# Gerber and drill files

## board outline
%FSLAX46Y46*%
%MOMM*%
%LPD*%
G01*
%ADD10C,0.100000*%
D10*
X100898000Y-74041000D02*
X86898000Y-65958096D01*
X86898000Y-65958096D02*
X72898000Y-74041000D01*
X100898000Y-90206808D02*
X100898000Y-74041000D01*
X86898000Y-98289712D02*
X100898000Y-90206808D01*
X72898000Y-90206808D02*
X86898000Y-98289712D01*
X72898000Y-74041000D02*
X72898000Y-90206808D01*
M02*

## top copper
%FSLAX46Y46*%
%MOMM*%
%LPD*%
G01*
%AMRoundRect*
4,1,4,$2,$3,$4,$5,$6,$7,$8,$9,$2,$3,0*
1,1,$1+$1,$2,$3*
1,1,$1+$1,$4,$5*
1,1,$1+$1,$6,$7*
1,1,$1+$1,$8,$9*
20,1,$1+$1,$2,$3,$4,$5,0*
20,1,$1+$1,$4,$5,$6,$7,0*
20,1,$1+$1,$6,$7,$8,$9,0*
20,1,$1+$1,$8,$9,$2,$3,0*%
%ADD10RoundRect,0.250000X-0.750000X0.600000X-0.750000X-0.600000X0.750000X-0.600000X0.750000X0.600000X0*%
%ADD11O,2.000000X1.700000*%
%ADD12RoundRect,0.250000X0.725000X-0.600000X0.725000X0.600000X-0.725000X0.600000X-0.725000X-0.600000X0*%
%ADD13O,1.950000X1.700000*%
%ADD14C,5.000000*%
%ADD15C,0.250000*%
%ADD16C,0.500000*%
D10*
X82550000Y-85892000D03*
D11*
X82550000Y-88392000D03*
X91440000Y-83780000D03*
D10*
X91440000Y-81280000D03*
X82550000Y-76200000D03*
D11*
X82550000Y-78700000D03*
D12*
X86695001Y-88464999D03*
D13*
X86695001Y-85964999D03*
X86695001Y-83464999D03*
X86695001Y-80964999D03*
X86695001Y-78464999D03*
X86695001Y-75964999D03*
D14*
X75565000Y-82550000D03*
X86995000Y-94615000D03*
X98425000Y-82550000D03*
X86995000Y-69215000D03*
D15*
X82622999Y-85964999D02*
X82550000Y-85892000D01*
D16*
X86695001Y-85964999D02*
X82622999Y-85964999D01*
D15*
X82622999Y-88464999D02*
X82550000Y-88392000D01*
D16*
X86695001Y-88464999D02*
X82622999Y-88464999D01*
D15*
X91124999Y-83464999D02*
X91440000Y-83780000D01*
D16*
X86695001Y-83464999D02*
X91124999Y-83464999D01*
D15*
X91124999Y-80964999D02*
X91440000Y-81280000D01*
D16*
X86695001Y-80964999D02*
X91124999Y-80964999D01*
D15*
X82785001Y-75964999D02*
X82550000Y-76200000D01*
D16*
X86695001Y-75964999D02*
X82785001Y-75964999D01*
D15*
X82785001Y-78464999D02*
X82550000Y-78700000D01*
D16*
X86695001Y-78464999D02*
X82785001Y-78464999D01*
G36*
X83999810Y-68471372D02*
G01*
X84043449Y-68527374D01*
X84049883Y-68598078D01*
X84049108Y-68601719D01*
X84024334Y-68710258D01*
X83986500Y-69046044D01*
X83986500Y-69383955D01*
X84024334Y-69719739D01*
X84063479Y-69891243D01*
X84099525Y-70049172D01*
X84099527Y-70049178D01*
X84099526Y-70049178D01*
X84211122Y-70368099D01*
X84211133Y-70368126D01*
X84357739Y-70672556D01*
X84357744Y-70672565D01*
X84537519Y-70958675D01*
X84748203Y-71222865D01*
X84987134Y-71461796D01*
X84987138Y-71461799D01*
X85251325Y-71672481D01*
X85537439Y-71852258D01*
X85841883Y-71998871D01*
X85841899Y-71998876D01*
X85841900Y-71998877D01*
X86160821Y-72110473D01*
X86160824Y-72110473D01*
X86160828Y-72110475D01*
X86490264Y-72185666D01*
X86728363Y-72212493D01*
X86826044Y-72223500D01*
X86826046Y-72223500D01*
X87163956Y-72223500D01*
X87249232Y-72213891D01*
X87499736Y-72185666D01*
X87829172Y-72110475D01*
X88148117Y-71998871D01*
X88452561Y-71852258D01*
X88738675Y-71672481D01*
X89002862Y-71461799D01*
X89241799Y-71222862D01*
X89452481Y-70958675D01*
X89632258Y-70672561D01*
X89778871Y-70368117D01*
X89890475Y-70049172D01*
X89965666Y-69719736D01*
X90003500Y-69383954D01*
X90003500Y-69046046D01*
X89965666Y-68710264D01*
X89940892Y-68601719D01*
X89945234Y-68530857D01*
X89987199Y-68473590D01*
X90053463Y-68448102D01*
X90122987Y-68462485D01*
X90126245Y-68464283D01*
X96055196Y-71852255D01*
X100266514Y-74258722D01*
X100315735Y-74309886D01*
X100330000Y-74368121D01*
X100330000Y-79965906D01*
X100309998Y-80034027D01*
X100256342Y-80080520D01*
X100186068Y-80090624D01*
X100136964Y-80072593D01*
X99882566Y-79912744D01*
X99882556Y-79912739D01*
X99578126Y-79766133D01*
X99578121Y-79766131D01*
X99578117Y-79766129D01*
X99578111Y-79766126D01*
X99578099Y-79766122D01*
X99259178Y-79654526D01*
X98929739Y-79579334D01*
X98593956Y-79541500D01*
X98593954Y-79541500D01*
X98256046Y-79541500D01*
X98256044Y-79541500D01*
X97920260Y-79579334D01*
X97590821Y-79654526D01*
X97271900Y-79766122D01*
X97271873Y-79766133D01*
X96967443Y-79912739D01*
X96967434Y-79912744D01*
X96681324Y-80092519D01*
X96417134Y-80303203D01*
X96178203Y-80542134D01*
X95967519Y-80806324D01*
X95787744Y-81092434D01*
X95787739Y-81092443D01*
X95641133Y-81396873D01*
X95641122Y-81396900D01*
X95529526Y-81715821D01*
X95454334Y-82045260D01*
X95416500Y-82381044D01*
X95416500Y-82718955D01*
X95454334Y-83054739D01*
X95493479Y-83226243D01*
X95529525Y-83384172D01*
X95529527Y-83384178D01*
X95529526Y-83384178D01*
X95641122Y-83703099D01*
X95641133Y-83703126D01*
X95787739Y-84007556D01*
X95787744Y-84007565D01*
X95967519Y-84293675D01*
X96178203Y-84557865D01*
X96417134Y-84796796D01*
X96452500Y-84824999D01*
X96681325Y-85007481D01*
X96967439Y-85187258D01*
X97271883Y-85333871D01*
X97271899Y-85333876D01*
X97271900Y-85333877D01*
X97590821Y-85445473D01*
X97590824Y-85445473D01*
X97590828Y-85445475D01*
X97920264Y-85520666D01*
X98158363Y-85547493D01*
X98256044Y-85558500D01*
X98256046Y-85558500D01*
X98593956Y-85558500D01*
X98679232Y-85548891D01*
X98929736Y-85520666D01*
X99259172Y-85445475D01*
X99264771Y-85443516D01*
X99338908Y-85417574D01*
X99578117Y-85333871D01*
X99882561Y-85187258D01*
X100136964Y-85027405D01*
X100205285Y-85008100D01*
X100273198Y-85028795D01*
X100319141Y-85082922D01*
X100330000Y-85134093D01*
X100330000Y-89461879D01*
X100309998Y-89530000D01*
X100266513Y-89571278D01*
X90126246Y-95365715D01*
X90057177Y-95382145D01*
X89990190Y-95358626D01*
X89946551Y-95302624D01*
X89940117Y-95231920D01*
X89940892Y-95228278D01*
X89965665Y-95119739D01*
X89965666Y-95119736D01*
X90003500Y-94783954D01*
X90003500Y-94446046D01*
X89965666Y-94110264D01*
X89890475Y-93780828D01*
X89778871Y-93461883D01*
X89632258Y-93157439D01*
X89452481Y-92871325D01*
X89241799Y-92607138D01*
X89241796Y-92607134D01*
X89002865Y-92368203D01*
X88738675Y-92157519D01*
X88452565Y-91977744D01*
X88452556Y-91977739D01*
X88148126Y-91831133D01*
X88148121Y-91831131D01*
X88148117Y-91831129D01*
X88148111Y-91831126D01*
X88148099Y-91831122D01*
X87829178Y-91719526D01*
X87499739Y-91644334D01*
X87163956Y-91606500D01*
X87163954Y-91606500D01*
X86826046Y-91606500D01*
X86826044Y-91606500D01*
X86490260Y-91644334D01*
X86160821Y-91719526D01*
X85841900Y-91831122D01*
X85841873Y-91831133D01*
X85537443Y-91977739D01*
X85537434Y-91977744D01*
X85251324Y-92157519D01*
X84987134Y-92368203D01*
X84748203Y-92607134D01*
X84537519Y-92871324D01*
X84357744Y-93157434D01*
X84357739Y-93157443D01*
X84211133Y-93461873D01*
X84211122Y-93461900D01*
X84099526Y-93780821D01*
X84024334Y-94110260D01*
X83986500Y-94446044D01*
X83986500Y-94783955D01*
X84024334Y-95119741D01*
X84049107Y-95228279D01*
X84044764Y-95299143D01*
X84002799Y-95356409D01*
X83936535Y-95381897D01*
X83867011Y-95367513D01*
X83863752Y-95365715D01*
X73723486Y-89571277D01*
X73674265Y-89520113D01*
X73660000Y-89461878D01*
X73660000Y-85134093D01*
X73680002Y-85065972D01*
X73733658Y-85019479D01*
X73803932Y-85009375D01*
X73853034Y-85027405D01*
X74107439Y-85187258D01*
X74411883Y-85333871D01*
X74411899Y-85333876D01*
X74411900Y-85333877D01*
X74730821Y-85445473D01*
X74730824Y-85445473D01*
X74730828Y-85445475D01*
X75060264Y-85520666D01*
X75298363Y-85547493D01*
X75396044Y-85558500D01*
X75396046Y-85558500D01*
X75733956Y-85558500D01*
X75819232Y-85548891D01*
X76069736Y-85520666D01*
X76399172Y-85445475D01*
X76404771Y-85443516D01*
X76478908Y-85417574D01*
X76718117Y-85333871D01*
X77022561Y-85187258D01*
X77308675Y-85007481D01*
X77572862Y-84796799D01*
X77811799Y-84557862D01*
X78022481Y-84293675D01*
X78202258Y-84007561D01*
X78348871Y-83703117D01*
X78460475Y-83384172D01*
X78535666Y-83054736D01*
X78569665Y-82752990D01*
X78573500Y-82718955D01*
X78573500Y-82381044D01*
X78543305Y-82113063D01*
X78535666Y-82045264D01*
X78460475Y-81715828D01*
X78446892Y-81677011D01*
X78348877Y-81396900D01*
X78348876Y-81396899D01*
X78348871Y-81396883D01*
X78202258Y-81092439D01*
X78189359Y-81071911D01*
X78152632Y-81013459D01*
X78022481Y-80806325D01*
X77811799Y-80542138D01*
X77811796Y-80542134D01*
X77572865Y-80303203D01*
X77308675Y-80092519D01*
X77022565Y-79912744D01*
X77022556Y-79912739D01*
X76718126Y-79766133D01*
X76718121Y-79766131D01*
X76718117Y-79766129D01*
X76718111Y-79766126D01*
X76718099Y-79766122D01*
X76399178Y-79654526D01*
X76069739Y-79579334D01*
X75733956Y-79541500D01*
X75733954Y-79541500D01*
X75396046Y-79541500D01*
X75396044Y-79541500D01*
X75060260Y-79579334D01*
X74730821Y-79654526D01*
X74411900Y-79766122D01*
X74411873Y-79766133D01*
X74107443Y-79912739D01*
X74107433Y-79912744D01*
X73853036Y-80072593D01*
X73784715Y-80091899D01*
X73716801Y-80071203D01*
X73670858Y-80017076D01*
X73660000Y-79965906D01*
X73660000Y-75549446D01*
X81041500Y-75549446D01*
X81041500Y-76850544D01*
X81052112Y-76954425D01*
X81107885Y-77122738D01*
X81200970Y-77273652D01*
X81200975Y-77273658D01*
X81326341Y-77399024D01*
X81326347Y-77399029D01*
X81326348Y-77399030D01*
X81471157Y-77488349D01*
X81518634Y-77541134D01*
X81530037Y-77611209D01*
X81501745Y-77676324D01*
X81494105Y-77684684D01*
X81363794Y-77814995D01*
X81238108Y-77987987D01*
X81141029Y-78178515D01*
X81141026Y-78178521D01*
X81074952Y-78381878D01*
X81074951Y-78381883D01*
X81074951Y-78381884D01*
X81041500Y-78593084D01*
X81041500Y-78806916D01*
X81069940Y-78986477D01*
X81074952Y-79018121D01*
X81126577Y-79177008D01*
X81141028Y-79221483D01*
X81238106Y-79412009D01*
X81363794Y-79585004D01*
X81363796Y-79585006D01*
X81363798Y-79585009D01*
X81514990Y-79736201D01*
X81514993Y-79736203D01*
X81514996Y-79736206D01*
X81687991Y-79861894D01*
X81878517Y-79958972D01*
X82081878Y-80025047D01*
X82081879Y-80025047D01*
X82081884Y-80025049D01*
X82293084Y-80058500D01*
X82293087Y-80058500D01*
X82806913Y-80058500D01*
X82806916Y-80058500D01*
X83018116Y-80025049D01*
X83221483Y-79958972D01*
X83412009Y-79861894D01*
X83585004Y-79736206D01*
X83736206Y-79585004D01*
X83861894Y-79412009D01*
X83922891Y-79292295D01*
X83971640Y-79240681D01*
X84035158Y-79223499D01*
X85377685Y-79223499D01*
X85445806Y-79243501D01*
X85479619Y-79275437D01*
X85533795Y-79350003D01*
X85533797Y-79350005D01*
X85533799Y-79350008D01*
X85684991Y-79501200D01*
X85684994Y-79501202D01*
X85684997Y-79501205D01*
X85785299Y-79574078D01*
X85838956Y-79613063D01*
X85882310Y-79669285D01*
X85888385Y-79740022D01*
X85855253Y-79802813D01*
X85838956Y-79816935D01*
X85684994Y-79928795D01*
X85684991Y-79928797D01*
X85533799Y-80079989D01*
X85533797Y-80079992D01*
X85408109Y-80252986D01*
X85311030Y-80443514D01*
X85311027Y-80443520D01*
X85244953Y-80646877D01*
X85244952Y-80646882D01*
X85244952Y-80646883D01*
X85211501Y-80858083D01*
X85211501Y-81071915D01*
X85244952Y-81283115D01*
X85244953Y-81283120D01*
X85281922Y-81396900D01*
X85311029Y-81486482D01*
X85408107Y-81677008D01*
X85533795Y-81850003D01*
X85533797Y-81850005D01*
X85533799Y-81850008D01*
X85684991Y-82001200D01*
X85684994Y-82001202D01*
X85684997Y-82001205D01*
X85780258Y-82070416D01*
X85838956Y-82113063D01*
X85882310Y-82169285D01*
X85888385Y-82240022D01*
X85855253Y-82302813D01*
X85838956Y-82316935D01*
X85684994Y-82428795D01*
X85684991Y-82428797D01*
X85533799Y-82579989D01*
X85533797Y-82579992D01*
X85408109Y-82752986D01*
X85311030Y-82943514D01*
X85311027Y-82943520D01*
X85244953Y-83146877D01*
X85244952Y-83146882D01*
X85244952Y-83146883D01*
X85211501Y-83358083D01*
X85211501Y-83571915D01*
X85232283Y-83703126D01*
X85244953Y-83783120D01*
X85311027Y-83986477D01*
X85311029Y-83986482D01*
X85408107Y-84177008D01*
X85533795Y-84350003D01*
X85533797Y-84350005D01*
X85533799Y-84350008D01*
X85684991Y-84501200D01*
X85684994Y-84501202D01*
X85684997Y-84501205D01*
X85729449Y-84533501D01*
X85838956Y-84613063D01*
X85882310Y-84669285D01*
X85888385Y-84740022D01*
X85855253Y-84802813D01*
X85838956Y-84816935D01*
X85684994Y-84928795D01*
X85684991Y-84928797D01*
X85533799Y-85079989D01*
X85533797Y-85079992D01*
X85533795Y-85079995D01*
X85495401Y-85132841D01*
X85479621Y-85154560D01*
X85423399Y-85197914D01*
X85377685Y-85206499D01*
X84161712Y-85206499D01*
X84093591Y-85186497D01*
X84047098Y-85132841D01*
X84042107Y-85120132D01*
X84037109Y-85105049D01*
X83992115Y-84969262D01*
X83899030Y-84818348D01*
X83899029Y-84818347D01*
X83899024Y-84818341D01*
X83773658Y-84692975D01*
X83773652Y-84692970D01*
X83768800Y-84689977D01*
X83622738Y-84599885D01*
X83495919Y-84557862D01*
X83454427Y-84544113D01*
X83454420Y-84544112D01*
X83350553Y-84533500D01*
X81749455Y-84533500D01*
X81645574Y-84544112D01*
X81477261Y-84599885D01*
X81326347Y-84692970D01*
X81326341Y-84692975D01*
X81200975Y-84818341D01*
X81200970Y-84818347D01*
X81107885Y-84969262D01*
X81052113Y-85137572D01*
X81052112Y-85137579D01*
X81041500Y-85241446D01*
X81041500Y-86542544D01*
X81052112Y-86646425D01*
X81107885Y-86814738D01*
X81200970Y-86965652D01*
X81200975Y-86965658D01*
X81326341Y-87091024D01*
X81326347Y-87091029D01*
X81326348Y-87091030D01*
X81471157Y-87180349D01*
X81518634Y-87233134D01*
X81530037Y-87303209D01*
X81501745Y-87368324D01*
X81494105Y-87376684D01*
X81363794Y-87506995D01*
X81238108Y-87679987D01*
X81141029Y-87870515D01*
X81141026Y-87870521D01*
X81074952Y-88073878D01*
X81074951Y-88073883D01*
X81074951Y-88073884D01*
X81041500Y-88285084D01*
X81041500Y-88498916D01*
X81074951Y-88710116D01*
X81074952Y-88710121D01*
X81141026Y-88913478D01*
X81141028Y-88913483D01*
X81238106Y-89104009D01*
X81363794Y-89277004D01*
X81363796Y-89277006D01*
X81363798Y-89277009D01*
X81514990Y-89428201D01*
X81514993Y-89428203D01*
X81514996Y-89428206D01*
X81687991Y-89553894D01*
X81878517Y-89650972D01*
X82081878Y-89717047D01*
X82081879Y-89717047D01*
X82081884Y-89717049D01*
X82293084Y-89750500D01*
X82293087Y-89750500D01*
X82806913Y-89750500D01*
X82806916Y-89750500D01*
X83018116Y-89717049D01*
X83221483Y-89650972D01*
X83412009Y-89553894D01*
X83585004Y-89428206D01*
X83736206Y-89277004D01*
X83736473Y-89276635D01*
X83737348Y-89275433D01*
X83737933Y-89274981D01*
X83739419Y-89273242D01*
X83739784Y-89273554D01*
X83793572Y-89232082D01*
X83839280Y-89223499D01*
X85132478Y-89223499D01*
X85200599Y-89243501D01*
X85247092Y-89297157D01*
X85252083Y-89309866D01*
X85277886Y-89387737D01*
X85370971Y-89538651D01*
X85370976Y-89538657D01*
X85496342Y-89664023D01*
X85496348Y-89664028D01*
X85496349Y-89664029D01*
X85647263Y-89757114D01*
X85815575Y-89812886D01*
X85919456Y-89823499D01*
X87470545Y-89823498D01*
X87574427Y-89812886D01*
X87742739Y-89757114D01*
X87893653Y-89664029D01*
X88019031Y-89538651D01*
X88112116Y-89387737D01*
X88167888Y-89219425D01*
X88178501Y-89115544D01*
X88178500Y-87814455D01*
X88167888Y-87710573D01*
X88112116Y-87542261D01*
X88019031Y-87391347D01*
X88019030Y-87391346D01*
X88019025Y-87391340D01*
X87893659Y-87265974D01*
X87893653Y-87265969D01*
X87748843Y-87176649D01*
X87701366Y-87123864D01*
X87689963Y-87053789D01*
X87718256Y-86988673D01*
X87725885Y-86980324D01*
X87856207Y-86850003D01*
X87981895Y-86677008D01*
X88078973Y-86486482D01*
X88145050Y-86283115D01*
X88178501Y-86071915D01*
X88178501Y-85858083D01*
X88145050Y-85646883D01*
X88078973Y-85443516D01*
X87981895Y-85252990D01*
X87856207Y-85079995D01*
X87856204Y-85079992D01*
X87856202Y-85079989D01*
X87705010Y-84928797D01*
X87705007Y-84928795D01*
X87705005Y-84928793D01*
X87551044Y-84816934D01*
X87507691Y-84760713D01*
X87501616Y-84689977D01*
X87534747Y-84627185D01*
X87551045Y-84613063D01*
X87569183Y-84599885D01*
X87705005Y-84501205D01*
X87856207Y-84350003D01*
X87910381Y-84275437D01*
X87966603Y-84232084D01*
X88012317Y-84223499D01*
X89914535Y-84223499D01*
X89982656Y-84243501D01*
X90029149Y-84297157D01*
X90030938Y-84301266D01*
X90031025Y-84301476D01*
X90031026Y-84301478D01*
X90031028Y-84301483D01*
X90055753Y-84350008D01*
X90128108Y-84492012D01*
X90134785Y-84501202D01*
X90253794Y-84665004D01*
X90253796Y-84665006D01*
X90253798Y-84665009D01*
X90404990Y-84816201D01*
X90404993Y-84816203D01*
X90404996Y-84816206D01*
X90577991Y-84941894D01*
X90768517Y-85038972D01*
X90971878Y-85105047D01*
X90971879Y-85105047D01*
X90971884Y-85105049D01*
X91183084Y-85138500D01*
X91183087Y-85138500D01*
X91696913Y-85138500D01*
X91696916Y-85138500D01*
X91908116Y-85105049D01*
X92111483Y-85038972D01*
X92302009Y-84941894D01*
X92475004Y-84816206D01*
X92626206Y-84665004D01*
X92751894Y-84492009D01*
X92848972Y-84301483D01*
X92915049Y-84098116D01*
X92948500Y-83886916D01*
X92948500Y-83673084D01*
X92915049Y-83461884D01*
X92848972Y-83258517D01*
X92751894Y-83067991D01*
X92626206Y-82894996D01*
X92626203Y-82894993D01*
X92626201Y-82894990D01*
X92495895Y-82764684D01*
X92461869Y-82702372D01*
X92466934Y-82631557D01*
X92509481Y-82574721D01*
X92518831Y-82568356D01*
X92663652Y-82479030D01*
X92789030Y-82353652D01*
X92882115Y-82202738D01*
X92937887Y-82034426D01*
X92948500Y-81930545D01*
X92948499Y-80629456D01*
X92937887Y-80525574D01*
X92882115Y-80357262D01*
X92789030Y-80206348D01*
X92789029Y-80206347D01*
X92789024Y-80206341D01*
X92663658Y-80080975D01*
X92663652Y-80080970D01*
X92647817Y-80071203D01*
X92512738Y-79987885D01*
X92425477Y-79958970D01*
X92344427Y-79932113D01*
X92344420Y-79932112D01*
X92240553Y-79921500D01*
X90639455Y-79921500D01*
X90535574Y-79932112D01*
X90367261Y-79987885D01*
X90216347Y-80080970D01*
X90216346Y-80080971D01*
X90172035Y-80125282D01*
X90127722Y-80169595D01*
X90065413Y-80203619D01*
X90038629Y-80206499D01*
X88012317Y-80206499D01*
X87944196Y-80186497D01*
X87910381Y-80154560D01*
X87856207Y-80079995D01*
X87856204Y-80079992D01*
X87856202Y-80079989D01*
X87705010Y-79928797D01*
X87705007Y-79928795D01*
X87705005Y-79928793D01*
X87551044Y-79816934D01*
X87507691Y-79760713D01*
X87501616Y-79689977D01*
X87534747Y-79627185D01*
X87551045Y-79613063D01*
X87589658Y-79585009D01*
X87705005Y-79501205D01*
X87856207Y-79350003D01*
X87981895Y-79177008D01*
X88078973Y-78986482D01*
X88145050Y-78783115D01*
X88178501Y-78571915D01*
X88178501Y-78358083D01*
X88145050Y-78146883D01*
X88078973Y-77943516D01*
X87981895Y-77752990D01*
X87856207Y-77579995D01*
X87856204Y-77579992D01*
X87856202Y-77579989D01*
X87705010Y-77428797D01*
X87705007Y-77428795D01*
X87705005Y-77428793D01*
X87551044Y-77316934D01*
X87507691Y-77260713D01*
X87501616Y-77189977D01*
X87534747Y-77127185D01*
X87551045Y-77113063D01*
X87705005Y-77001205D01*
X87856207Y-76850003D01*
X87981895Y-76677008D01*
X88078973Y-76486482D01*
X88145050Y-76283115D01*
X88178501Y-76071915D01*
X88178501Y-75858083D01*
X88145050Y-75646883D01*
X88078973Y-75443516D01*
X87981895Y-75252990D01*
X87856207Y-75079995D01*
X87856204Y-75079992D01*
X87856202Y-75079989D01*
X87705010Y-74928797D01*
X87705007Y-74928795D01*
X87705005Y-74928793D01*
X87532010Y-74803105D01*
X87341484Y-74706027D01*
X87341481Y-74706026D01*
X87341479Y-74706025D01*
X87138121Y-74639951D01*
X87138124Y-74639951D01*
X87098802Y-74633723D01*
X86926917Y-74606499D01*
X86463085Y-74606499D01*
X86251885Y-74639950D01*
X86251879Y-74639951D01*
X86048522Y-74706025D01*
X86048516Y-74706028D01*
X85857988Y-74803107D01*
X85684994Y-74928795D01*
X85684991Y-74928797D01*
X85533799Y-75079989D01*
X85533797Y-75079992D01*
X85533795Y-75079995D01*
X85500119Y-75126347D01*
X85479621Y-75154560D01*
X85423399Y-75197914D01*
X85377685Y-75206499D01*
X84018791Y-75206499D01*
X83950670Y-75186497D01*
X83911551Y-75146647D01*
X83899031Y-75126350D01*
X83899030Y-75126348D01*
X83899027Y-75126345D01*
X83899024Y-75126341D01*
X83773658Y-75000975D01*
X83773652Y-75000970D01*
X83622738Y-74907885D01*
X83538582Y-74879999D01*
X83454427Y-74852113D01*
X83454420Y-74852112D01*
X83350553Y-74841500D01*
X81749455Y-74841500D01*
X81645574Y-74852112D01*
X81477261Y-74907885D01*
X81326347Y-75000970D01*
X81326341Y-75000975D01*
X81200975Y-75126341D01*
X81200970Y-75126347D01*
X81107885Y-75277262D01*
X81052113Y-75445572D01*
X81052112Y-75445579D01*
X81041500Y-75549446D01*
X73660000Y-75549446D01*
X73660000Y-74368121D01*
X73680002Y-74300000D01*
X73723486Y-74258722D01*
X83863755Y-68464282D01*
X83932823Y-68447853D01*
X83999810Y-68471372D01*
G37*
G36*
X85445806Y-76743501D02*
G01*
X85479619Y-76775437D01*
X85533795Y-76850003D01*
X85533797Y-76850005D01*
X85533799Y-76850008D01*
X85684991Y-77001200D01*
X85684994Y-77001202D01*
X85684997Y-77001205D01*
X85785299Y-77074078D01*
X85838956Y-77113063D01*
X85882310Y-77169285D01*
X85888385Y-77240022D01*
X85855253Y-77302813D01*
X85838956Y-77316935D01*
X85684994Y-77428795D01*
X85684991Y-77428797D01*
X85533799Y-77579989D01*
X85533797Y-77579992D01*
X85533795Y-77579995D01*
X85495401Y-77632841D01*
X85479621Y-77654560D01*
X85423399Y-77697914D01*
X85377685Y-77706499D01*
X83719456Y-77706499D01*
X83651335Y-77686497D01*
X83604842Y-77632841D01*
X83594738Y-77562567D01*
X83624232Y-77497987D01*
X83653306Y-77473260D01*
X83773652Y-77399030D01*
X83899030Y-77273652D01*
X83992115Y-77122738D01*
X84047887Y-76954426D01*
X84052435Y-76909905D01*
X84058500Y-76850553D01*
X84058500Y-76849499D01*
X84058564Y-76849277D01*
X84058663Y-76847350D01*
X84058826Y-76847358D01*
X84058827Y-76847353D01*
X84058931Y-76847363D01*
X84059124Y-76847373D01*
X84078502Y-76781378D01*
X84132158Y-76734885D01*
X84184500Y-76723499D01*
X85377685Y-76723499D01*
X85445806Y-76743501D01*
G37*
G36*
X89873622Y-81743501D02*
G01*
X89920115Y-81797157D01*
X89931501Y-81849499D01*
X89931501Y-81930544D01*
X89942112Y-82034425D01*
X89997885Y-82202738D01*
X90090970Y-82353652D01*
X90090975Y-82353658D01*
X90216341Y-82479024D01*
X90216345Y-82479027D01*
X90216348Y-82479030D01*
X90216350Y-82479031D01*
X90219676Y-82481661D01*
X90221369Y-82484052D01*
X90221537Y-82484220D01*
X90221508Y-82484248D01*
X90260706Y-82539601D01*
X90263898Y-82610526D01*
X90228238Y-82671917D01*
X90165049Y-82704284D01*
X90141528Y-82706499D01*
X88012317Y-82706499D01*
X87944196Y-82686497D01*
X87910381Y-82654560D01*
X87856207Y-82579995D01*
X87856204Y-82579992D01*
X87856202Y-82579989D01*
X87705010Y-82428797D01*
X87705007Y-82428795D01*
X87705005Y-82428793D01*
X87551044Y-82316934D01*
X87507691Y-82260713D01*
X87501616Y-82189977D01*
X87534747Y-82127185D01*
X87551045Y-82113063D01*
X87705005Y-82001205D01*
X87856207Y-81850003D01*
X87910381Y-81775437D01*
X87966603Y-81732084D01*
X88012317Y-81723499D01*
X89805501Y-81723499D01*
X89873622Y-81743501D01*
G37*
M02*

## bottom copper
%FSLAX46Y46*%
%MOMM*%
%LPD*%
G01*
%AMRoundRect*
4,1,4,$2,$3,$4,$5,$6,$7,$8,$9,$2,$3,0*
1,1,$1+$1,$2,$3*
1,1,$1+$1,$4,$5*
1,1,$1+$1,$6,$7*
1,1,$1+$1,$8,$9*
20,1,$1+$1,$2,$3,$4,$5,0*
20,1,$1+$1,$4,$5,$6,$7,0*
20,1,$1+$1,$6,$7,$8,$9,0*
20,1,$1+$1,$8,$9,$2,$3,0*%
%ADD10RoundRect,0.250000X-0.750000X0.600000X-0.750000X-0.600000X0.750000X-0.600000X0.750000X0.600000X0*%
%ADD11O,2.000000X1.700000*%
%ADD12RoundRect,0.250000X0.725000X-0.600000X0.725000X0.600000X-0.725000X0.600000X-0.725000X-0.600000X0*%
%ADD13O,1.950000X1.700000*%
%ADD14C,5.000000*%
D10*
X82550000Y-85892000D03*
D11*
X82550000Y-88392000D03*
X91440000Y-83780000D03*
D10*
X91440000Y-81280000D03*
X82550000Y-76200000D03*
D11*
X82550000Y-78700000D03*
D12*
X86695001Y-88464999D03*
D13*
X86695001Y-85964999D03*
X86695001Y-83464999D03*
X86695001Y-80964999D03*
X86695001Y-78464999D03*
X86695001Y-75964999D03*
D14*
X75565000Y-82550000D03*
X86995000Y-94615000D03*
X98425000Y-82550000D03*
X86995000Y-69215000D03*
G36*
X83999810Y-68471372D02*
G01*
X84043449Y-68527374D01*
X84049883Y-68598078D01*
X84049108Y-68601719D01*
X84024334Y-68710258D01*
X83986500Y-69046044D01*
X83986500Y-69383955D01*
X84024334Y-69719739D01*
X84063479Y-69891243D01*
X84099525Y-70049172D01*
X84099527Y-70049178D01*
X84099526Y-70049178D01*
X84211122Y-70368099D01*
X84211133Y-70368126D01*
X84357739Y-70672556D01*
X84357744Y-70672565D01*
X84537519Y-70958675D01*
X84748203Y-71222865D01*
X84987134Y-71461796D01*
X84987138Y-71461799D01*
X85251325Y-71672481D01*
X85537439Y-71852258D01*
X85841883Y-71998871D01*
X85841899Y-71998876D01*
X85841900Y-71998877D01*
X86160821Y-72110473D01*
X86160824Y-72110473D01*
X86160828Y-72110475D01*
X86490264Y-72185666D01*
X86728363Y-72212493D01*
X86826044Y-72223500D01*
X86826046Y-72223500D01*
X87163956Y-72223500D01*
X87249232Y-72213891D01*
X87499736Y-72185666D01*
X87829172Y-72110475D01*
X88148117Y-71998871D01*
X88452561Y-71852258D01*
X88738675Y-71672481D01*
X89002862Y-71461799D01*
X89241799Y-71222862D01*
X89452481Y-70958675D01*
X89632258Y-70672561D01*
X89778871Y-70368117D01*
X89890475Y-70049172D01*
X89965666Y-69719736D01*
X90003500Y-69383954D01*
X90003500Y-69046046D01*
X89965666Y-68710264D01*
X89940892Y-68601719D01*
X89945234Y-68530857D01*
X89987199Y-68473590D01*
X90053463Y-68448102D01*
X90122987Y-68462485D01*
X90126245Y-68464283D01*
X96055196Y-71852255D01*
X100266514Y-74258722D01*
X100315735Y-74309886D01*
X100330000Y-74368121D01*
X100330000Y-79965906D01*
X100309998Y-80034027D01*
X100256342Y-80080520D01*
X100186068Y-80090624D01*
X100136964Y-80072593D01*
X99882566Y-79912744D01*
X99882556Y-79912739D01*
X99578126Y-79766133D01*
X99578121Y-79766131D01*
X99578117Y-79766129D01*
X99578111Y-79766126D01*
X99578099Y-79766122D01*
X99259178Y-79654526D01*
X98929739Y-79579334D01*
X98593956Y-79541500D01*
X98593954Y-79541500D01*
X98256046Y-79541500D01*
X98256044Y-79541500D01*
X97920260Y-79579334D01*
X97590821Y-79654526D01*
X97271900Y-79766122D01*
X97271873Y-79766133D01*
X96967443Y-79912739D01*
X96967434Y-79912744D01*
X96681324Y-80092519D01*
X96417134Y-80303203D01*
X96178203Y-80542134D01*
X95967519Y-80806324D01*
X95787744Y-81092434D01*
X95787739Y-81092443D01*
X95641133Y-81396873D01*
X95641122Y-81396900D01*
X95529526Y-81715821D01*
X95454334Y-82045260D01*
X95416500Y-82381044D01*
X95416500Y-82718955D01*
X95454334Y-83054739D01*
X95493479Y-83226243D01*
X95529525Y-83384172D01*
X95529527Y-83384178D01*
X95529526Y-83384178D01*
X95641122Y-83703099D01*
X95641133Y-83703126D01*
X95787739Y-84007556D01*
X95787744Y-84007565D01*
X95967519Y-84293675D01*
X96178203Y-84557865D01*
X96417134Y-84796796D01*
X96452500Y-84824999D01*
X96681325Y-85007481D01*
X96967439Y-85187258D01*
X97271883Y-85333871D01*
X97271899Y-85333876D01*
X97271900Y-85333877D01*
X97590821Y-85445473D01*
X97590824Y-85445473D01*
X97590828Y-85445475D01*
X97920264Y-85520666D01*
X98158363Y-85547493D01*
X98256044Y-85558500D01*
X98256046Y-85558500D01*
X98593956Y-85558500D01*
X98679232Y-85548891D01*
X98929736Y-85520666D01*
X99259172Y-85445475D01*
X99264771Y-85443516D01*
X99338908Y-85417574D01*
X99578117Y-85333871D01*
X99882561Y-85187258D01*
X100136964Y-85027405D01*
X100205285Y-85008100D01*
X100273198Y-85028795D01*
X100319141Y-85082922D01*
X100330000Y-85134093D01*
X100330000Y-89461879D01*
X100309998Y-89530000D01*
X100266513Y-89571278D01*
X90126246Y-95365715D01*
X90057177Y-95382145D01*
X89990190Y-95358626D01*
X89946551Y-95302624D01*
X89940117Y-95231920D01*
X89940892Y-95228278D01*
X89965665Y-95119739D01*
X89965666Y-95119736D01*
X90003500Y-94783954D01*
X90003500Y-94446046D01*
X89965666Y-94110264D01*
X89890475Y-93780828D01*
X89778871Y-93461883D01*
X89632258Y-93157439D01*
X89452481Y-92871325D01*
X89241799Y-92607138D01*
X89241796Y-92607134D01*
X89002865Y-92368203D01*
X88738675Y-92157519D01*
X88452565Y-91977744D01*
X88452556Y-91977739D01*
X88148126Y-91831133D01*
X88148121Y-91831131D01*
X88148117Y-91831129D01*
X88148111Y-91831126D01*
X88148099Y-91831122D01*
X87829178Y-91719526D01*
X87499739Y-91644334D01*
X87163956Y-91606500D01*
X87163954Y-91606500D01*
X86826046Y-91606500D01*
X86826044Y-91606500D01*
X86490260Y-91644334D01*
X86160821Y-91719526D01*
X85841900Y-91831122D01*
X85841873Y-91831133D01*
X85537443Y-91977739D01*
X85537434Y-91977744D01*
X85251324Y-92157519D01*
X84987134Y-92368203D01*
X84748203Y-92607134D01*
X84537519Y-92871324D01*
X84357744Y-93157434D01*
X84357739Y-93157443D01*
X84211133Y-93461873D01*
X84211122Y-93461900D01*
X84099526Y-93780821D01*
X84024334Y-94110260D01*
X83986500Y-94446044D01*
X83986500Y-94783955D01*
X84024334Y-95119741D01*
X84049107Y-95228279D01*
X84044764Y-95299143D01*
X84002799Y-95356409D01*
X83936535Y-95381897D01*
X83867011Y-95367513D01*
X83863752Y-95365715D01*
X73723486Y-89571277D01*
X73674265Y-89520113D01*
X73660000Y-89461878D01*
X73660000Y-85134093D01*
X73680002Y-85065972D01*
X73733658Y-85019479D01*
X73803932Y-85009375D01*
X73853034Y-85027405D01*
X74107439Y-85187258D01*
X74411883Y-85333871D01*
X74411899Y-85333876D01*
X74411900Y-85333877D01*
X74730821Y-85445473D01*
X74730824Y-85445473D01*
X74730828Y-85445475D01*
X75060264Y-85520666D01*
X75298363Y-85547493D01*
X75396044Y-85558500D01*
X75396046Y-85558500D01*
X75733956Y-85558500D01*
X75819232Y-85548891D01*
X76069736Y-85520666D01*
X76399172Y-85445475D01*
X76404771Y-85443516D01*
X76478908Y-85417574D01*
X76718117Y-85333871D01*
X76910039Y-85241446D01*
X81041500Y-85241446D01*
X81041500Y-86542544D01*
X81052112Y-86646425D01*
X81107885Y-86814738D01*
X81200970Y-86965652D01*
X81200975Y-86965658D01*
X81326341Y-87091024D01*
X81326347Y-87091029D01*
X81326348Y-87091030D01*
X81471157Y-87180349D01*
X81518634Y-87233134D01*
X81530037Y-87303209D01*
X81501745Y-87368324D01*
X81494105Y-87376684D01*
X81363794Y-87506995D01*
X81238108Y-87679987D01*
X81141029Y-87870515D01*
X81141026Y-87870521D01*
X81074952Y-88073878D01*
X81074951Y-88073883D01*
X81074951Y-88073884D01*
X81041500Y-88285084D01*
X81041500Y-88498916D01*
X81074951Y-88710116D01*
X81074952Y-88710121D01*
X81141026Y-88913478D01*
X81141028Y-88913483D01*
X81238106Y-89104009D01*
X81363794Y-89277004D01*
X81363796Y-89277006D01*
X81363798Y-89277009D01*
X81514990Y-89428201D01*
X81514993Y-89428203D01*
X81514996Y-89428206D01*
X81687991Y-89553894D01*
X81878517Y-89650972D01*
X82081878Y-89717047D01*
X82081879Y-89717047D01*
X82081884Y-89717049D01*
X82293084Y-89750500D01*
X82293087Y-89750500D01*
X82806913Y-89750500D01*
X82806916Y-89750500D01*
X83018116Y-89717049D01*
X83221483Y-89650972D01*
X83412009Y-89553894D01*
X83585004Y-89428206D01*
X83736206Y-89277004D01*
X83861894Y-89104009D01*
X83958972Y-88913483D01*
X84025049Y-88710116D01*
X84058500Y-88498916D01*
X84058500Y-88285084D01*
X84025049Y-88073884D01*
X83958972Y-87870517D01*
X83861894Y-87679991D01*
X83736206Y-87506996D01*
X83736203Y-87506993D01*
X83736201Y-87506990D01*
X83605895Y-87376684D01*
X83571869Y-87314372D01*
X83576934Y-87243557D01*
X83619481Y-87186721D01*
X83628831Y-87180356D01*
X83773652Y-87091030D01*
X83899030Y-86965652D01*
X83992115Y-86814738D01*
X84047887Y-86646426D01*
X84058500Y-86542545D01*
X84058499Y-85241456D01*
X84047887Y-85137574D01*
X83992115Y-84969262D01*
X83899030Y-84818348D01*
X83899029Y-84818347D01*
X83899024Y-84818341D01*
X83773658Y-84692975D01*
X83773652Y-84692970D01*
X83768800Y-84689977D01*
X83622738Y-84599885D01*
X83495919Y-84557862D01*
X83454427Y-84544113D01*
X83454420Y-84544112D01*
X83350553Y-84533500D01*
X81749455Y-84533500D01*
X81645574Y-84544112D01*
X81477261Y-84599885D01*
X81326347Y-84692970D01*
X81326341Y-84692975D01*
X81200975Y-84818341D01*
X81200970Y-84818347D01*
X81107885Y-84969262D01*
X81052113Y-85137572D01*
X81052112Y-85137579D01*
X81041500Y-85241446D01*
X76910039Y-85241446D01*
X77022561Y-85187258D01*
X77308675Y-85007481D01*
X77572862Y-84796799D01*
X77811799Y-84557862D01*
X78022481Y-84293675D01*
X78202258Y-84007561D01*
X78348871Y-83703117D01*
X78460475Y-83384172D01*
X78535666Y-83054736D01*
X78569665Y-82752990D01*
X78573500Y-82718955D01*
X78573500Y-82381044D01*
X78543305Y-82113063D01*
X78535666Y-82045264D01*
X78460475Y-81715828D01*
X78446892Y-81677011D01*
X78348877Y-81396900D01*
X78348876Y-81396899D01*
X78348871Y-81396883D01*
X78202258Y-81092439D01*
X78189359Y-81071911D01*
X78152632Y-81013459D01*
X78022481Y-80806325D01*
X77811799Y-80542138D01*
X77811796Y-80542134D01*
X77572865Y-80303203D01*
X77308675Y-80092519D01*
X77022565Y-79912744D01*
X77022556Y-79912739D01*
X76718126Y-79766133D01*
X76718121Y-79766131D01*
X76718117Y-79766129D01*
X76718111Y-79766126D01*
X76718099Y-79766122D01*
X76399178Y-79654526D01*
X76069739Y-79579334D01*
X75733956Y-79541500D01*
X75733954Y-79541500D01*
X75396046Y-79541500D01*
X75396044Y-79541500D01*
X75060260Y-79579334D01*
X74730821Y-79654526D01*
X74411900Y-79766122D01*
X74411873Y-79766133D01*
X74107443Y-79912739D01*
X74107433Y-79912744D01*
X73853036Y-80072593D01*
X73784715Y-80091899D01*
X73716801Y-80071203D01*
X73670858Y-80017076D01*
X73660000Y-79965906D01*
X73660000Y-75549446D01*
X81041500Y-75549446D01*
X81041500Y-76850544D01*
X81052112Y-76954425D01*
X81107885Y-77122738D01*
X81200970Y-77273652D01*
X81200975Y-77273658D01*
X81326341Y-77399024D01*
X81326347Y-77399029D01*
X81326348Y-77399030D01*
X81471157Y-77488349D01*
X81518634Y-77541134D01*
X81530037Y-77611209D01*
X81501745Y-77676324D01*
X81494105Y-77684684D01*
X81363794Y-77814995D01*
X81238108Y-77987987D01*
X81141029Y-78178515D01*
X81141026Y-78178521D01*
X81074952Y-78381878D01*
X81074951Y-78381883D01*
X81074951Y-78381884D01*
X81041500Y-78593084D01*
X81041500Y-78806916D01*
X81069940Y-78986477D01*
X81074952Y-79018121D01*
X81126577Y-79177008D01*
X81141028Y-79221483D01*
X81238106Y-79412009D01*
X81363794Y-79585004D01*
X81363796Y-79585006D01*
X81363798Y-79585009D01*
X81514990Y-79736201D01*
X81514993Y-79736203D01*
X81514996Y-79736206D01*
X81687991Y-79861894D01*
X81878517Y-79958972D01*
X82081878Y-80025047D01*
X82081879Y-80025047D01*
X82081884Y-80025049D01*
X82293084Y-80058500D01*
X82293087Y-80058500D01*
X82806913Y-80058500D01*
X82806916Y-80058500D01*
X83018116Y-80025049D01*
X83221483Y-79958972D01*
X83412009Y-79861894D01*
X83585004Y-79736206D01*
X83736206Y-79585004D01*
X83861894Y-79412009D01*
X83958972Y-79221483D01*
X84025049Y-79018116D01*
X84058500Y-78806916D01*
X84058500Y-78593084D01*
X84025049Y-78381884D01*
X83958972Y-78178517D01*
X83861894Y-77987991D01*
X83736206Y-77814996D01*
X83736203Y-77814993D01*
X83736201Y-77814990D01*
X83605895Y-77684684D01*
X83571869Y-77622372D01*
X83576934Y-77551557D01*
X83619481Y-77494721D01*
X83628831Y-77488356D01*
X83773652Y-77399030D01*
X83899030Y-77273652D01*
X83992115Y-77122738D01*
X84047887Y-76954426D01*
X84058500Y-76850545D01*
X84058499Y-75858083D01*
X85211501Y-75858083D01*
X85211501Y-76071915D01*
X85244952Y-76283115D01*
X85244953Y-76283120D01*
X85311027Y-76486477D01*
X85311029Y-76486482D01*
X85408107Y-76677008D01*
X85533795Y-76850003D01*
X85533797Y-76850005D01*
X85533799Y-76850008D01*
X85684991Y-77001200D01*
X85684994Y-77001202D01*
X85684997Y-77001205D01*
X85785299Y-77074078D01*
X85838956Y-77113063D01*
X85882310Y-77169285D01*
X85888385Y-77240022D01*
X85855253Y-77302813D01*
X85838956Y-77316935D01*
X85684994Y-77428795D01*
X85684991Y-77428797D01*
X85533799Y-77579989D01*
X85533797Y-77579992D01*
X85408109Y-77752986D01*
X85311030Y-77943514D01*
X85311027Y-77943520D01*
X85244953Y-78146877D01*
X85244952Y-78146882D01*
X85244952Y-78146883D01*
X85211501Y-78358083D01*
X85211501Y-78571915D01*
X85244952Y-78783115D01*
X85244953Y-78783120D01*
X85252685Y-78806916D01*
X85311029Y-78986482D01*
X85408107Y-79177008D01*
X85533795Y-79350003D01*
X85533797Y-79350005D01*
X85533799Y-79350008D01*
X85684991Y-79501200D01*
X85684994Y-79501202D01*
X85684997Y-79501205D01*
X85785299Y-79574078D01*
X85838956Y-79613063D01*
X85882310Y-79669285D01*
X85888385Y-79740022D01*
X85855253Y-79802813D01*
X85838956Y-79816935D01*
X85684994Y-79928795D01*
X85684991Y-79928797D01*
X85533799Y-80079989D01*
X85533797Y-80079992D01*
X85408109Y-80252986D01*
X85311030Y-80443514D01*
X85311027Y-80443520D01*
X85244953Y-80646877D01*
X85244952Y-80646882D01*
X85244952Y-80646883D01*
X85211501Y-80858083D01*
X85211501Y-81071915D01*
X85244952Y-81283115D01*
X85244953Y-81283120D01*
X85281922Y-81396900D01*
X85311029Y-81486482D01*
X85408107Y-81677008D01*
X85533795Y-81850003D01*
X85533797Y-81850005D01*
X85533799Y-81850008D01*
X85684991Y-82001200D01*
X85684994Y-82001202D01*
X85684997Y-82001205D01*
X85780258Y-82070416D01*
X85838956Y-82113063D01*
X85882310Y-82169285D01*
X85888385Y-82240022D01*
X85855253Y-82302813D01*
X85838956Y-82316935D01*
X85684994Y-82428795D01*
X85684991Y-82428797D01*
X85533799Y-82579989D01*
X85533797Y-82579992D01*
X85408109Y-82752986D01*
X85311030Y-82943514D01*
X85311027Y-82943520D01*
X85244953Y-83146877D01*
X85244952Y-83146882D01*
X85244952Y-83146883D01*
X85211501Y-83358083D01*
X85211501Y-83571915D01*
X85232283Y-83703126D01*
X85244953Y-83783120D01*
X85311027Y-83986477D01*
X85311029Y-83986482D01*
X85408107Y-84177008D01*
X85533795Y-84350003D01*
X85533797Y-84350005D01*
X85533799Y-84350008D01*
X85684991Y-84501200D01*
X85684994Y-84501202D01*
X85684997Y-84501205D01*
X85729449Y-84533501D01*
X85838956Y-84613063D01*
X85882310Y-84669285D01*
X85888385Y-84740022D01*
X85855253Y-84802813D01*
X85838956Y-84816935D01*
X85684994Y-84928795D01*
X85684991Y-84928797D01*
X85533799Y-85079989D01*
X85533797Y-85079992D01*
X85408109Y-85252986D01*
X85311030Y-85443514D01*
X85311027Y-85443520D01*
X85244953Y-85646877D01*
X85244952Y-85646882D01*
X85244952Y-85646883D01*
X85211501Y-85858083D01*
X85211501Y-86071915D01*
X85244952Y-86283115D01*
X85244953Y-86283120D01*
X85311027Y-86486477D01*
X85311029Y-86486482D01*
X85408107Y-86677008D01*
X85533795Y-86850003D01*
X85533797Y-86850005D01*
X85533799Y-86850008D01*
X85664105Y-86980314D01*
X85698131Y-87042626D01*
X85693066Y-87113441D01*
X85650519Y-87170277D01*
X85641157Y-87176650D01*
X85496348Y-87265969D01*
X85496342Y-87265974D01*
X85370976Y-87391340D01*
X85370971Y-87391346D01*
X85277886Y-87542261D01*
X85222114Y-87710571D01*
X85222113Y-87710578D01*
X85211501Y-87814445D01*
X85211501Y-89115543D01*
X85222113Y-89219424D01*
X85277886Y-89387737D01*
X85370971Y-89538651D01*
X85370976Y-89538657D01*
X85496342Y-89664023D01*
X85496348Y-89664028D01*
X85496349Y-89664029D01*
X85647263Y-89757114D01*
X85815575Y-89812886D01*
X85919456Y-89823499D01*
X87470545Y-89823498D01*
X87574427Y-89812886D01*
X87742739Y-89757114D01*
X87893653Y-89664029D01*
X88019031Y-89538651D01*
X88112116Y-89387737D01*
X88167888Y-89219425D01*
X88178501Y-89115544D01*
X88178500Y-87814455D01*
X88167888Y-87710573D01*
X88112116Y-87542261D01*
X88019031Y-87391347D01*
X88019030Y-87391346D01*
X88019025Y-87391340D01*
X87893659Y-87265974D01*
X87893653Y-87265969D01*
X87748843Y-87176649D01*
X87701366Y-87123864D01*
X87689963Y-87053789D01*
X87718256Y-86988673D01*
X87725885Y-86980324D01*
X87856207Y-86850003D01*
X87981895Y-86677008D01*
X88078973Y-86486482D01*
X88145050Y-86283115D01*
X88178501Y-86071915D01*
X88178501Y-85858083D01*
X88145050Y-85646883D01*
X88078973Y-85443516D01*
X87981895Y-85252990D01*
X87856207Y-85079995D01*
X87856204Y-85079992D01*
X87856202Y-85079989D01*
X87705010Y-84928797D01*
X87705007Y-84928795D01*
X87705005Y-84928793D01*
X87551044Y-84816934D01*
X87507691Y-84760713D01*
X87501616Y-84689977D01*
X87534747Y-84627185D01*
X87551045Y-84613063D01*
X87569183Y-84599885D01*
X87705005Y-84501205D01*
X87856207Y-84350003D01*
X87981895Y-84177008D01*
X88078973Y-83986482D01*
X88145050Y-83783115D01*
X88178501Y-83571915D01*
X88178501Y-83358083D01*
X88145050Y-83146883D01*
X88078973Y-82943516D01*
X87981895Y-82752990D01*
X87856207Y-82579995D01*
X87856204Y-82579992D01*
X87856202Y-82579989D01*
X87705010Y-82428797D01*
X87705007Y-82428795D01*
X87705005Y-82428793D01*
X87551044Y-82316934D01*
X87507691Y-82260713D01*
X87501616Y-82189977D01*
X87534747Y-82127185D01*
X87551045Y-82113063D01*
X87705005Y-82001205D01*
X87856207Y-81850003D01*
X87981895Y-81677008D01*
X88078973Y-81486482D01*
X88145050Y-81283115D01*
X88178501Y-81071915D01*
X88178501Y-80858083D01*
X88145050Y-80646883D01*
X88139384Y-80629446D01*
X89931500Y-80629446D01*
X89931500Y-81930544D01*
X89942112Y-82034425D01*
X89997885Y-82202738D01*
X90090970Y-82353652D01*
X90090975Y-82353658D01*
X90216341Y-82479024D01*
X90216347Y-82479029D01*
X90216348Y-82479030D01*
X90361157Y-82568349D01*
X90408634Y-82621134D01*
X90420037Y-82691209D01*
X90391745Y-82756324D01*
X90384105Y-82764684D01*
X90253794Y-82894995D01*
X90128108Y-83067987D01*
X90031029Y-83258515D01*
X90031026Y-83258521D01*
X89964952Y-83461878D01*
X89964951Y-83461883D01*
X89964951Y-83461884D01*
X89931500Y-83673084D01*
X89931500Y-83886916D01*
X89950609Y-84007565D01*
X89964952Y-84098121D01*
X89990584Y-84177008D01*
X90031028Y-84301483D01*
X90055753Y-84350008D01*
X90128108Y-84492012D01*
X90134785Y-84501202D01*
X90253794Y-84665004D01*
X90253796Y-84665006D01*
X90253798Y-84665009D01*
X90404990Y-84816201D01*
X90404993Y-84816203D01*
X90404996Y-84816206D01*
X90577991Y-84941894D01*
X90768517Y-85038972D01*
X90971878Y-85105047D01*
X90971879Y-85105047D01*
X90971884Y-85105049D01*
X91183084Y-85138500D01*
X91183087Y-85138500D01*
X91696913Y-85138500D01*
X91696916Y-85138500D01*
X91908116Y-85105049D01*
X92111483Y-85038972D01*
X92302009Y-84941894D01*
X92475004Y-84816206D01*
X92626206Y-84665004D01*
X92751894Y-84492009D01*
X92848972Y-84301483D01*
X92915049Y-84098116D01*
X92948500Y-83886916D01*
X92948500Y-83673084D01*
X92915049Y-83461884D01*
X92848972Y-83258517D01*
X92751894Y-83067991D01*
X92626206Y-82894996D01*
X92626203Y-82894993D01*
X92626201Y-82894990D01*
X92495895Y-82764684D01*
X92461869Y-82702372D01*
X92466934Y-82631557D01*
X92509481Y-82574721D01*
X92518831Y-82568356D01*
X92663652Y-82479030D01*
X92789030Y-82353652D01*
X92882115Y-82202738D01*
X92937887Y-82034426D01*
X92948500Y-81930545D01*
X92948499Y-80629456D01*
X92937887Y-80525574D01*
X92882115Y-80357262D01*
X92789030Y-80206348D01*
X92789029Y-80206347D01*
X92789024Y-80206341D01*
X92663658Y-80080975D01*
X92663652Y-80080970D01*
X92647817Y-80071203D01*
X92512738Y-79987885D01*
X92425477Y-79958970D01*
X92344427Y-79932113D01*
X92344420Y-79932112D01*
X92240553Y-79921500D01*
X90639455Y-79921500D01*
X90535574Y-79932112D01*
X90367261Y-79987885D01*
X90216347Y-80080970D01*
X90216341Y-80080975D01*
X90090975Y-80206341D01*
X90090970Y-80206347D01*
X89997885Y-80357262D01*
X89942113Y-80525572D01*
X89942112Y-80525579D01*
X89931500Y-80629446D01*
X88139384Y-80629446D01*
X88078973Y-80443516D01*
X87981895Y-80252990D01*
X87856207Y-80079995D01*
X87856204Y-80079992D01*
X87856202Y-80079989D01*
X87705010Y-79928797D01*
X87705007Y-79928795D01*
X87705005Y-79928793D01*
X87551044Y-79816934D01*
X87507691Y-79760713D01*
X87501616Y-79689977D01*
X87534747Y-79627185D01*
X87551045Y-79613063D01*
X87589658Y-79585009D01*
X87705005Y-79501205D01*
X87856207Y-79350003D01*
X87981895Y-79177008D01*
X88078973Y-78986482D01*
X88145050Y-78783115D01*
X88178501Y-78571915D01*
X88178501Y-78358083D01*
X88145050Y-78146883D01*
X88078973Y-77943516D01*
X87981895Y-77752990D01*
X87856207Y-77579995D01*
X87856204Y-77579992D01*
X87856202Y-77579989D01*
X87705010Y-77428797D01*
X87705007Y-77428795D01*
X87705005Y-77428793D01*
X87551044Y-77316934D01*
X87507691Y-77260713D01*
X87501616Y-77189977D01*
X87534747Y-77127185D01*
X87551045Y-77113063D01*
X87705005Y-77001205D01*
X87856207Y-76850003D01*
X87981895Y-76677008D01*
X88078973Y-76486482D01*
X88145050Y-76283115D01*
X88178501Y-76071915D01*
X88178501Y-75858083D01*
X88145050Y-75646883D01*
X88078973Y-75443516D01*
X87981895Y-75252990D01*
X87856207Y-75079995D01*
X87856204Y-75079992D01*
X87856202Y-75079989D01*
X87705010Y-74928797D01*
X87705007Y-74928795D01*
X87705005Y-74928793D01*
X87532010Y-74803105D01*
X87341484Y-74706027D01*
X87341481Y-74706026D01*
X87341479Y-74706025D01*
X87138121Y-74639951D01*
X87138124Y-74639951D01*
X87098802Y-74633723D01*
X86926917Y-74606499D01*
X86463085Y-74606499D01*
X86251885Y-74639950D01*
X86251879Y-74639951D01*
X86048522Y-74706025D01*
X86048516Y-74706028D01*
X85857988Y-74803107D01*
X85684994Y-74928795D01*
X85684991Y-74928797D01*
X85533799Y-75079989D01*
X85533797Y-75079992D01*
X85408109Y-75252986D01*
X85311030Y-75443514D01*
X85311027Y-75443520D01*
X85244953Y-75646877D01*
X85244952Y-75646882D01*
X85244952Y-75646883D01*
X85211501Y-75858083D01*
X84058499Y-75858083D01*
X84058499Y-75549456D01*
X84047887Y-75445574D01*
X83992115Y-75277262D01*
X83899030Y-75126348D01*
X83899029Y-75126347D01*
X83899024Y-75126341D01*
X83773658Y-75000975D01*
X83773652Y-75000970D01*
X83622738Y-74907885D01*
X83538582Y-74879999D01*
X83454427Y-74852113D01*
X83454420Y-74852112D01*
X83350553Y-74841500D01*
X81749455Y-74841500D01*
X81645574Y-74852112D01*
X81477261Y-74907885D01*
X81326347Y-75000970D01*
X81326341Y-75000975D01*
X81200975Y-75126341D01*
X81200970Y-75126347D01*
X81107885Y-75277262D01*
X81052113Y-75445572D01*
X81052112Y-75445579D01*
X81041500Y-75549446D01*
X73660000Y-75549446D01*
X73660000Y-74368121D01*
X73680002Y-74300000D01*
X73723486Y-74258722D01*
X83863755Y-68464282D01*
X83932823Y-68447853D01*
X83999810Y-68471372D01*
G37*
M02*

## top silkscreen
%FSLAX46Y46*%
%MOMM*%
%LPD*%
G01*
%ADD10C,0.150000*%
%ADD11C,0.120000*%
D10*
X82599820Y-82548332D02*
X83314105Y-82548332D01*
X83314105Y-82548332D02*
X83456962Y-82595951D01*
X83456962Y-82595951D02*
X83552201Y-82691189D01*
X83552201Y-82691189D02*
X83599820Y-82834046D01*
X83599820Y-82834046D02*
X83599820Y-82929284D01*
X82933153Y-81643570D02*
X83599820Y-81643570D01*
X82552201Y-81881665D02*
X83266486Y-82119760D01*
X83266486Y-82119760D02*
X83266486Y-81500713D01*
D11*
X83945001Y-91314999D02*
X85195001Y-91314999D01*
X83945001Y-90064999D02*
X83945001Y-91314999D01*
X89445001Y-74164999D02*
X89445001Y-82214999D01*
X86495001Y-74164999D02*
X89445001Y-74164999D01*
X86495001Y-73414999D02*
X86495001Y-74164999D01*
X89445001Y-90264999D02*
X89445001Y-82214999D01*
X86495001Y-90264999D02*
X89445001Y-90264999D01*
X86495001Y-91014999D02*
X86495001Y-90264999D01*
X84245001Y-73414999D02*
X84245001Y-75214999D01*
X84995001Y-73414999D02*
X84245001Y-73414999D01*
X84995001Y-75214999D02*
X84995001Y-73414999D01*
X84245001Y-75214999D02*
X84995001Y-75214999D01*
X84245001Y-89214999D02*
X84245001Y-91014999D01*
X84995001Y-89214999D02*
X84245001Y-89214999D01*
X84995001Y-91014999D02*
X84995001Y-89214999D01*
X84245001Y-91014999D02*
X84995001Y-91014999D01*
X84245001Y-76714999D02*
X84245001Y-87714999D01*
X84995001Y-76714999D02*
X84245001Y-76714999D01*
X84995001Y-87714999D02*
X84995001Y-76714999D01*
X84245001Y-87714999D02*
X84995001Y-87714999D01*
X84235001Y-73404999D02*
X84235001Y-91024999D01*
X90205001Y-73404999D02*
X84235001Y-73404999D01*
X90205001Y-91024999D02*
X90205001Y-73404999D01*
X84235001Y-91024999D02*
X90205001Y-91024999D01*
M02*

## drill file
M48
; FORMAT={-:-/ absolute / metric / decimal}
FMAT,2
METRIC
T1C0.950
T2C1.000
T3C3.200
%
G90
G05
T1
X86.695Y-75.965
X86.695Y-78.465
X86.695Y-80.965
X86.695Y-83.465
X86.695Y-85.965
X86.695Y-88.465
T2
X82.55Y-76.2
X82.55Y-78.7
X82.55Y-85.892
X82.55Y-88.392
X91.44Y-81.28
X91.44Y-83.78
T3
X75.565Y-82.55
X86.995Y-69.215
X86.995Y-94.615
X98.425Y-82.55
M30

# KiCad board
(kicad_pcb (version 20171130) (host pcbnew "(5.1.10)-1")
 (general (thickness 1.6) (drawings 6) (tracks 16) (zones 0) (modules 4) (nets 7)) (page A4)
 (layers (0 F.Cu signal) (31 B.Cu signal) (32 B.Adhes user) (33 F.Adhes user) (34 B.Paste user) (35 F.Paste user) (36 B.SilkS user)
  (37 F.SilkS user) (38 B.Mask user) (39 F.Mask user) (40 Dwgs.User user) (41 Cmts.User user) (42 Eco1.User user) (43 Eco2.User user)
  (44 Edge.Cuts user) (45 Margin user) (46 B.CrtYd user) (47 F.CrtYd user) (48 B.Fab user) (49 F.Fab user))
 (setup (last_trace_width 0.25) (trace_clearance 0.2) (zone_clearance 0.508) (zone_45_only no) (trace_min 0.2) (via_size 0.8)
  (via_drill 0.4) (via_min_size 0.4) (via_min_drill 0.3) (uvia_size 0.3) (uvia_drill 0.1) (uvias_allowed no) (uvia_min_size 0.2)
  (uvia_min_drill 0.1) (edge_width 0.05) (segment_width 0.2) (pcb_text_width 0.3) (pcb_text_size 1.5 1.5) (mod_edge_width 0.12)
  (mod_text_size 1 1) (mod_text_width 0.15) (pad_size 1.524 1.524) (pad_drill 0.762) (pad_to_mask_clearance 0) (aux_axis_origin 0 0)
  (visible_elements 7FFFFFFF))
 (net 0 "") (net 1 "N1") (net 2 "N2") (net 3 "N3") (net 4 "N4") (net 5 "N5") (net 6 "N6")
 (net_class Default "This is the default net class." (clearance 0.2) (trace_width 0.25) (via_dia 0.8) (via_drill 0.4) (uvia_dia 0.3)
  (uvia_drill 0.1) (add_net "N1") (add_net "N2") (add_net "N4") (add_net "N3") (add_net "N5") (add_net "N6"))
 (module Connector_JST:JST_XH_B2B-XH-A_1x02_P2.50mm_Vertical (layer B.Cu) (at 82.55 85.892 270)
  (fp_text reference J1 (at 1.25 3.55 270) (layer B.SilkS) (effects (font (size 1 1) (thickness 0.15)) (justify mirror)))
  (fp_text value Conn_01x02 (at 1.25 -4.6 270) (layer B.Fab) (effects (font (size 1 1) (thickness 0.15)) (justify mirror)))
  (pad 1 thru_hole roundrect (at 0 0 270) (size 1.7 2) (drill 1) (layers *.Cu *.Mask) (roundrect_rratio 0.1470588235294118) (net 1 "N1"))
  (pad 2 thru_hole oval (at 2.5 0 270) (size 1.7 2) (drill 1) (layers *.Cu *.Mask) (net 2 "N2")))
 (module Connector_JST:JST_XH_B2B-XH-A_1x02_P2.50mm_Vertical (layer B.Cu) (at 91.44 81.28 270)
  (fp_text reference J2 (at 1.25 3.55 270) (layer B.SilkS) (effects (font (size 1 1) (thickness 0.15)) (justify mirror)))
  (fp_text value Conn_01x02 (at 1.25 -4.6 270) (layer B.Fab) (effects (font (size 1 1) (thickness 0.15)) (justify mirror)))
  (pad 2 thru_hole oval (at 2.5 0 270) (size 1.7 2) (drill 1) (layers *.Cu *.Mask) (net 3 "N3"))
  (pad 1 thru_hole roundrect (at 0 0 270) (size 1.7 2) (drill 1) (layers *.Cu *.Mask) (roundrect_rratio 0.1470588235294118) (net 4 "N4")))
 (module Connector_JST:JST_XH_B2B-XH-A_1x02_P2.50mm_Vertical (layer B.Cu) (at 82.55 76.2 270)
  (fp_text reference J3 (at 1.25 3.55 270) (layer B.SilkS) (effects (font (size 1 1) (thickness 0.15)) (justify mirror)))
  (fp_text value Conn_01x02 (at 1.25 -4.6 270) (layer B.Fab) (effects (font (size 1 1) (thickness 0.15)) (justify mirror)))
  (pad 1 thru_hole roundrect (at 0 0 270) (size 1.7 2) (drill 1) (layers *.Cu *.Mask) (roundrect_rratio 0.1470588235294118) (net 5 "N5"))
  (pad 2 thru_hole oval (at 2.5 0 270) (size 1.7 2) (drill 1) (layers *.Cu *.Mask) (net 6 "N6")))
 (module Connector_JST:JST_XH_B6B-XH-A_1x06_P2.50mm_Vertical (layer F.Cu) (at 86.695001 88.464999 90)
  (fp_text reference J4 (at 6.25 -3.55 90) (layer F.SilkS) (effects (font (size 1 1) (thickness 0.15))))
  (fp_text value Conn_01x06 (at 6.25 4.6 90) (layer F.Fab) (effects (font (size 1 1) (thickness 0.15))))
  (fp_line (start -2.85 -2.75) (end -2.85 -1.5) (layer F.SilkS) (width 0.12))
  (fp_line (start -1.6 -2.75) (end -2.85 -2.75) (layer F.SilkS) (width 0.12))
  (fp_line (start 14.3 2.75) (end 6.25 2.75) (layer F.SilkS) (width 0.12))
  (fp_line (start 14.3 -0.2) (end 14.3 2.75) (layer F.SilkS) (width 0.12))
  (fp_line (start 15.05 -0.2) (end 14.3 -0.2) (layer F.SilkS) (width 0.12))
  (fp_line (start -1.8 2.75) (end 6.25 2.75) (layer F.SilkS) (width 0.12))
  (fp_line (start -1.8 -0.2) (end -1.8 2.75) (layer F.SilkS) (width 0.12))
  (fp_line (start -2.55 -0.2) (end -1.8 -0.2) (layer F.SilkS) (width 0.12))
  (fp_line (start 15.05 -2.45) (end 13.25 -2.45) (layer F.SilkS) (width 0.12))
  (fp_line (start 15.05 -1.7) (end 15.05 -2.45) (layer F.SilkS) (width 0.12))
  (fp_line (start 13.25 -1.7) (end 15.05 -1.7) (layer F.SilkS) (width 0.12))
  (fp_line (start 13.25 -2.45) (end 13.25 -1.7) (layer F.SilkS) (width 0.12))
  (fp_line (start -0.75 -2.45) (end -2.55 -2.45) (layer F.SilkS) (width 0.12))
  (fp_line (start -0.75 -1.7) (end -0.75 -2.45) (layer F.SilkS) (width 0.12))
  (fp_line (start -2.55 -1.7) (end -0.75 -1.7) (layer F.SilkS) (width 0.12))
  (fp_line (start -2.55 -2.45) (end -2.55 -1.7) (layer F.SilkS) (width 0.12))
  (fp_line (start 11.75 -2.45) (end 0.75 -2.45) (layer F.SilkS) (width 0.12))
  (fp_line (start 11.75 -1.7) (end 11.75 -2.45) (layer F.SilkS) (width 0.12))
  (fp_line (start 0.75 -1.7) (end 11.75 -1.7) (layer F.SilkS) (width 0.12))
  (fp_line (start 0.75 -2.45) (end 0.75 -1.7) (layer F.SilkS) (width 0.12))
  (fp_line (start 15.06 -2.46) (end -2.56 -2.46) (layer F.SilkS) (width 0.12))
  (fp_line (start 15.06 3.51) (end 15.06 -2.46) (layer F.SilkS) (width 0.12))
  (fp_line (start -2.56 3.51) (end 15.06 3.51) (layer F.SilkS) (width 0.12))
  (fp_line (start -2.56 -2.46) (end -2.56 3.51) (layer F.SilkS) (width 0.12))
  (pad 1 thru_hole roundrect (at 0 0 90) (size 1.7 1.95) (drill 0.95) (layers *.Cu *.Mask) (roundrect_rratio 0.1470588235294118)
   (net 2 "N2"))
  (pad 2 thru_hole oval (at 2.5 0 90) (size 1.7 1.95) (drill 0.95) (layers *.Cu *.Mask) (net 1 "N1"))
  (pad 3 thru_hole oval (at 5 0 90) (size 1.7 1.95) (drill 0.95) (layers *.Cu *.Mask) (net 3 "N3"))
  (pad 4 thru_hole oval (at 7.5 0 90) (size 1.7 1.95) (drill 0.95) (layers *.Cu *.Mask) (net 4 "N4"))
  (pad 5 thru_hole oval (at 10 0 90) (size 1.7 1.95) (drill 0.95) (layers *.Cu *.Mask) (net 6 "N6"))
  (pad 6 thru_hole oval (at 12.5 0 90) (size 1.7 1.95) (drill 0.95) (layers *.Cu *.Mask) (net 5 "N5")))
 (gr_line (start 100.898 74.041) (end 86.898 65.958096) (layer Edge.Cuts) (width 0.1))
 (gr_line (start 86.898 65.958096) (end 72.898 74.041) (layer Edge.Cuts) (width 0.1))
 (gr_line (start 100.898 90.206808) (end 100.898 74.041) (layer Edge.Cuts) (width 0.1))
 (gr_line (start 86.898 98.289712) (end 100.898 90.206808) (layer Edge.Cuts) (width 0.1))
 (gr_line (start 72.898 90.206808) (end 86.898 98.289712) (layer Edge.Cuts) (width 0.1))
 (gr_line (start 72.898 74.041) (end 72.898 90.206808) (layer Edge.Cuts) (width 0.1))
 (via (at 75.565 82.55) (size 5) (drill 3.2) (layers F.Cu B.Cu) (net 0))
 (via (at 86.995 94.615) (size 5) (drill 3.2) (layers F.Cu B.Cu) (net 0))
 (via (at 98.425 82.55) (size 5) (drill 3.2) (layers F.Cu B.Cu) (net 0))
 (via (at 86.995 69.215) (size 5) (drill 3.2) (layers F.Cu B.Cu) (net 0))
 (segment (start 82.622999 85.964999) (end 82.55 85.892) (width 0.25) (layer F.Cu) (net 1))
 (segment (start 86.695001 85.964999) (end 82.622999 85.964999) (width 0.5) (layer F.Cu) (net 1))
 (segment (start 82.622999 88.464999) (end 82.55 88.392) (width 0.25) (layer F.Cu) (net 2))
 (segment (start 86.695001 88.464999) (end 82.622999 88.464999) (width 0.5) (layer F.Cu) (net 2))
 (segment (start 91.124999 83.464999) (end 91.44 83.78) (width 0.25) (layer F.Cu) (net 3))
 (segment (start 86.695001 83.464999) (end 91.124999 83.464999) (width 0.5) (layer F.Cu) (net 3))
 (segment (start 91.124999 80.964999) (end 91.44 81.28) (width 0.25) (layer F.Cu) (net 4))
 (segment (start 86.695001 80.964999) (end 91.124999 80.964999) (width 0.5) (layer F.Cu) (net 4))
 (segment (start 82.785001 75.964999) (end 82.55 76.2) (width 0.25) (layer F.Cu) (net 5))
 (segment (start 86.695001 75.964999) (end 82.785001 75.964999) (width 0.5) (layer F.Cu) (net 5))
 (segment (start 82.785001 78.464999) (end 82.55 78.7) (width 0.25) (layer F.Cu) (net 6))
 (segment (start 86.695001 78.464999) (end 82.785001 78.464999) (width 0.5) (layer F.Cu) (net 6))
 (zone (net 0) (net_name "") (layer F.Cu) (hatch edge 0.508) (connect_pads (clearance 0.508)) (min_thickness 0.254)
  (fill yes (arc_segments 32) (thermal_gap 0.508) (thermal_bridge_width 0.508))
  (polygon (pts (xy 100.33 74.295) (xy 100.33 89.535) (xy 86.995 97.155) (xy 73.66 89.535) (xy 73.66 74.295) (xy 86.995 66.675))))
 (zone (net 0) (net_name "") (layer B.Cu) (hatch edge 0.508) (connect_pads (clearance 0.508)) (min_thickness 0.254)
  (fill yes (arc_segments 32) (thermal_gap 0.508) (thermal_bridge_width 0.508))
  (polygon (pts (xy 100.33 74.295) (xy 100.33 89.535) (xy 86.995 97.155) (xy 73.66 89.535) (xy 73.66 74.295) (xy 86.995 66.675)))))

